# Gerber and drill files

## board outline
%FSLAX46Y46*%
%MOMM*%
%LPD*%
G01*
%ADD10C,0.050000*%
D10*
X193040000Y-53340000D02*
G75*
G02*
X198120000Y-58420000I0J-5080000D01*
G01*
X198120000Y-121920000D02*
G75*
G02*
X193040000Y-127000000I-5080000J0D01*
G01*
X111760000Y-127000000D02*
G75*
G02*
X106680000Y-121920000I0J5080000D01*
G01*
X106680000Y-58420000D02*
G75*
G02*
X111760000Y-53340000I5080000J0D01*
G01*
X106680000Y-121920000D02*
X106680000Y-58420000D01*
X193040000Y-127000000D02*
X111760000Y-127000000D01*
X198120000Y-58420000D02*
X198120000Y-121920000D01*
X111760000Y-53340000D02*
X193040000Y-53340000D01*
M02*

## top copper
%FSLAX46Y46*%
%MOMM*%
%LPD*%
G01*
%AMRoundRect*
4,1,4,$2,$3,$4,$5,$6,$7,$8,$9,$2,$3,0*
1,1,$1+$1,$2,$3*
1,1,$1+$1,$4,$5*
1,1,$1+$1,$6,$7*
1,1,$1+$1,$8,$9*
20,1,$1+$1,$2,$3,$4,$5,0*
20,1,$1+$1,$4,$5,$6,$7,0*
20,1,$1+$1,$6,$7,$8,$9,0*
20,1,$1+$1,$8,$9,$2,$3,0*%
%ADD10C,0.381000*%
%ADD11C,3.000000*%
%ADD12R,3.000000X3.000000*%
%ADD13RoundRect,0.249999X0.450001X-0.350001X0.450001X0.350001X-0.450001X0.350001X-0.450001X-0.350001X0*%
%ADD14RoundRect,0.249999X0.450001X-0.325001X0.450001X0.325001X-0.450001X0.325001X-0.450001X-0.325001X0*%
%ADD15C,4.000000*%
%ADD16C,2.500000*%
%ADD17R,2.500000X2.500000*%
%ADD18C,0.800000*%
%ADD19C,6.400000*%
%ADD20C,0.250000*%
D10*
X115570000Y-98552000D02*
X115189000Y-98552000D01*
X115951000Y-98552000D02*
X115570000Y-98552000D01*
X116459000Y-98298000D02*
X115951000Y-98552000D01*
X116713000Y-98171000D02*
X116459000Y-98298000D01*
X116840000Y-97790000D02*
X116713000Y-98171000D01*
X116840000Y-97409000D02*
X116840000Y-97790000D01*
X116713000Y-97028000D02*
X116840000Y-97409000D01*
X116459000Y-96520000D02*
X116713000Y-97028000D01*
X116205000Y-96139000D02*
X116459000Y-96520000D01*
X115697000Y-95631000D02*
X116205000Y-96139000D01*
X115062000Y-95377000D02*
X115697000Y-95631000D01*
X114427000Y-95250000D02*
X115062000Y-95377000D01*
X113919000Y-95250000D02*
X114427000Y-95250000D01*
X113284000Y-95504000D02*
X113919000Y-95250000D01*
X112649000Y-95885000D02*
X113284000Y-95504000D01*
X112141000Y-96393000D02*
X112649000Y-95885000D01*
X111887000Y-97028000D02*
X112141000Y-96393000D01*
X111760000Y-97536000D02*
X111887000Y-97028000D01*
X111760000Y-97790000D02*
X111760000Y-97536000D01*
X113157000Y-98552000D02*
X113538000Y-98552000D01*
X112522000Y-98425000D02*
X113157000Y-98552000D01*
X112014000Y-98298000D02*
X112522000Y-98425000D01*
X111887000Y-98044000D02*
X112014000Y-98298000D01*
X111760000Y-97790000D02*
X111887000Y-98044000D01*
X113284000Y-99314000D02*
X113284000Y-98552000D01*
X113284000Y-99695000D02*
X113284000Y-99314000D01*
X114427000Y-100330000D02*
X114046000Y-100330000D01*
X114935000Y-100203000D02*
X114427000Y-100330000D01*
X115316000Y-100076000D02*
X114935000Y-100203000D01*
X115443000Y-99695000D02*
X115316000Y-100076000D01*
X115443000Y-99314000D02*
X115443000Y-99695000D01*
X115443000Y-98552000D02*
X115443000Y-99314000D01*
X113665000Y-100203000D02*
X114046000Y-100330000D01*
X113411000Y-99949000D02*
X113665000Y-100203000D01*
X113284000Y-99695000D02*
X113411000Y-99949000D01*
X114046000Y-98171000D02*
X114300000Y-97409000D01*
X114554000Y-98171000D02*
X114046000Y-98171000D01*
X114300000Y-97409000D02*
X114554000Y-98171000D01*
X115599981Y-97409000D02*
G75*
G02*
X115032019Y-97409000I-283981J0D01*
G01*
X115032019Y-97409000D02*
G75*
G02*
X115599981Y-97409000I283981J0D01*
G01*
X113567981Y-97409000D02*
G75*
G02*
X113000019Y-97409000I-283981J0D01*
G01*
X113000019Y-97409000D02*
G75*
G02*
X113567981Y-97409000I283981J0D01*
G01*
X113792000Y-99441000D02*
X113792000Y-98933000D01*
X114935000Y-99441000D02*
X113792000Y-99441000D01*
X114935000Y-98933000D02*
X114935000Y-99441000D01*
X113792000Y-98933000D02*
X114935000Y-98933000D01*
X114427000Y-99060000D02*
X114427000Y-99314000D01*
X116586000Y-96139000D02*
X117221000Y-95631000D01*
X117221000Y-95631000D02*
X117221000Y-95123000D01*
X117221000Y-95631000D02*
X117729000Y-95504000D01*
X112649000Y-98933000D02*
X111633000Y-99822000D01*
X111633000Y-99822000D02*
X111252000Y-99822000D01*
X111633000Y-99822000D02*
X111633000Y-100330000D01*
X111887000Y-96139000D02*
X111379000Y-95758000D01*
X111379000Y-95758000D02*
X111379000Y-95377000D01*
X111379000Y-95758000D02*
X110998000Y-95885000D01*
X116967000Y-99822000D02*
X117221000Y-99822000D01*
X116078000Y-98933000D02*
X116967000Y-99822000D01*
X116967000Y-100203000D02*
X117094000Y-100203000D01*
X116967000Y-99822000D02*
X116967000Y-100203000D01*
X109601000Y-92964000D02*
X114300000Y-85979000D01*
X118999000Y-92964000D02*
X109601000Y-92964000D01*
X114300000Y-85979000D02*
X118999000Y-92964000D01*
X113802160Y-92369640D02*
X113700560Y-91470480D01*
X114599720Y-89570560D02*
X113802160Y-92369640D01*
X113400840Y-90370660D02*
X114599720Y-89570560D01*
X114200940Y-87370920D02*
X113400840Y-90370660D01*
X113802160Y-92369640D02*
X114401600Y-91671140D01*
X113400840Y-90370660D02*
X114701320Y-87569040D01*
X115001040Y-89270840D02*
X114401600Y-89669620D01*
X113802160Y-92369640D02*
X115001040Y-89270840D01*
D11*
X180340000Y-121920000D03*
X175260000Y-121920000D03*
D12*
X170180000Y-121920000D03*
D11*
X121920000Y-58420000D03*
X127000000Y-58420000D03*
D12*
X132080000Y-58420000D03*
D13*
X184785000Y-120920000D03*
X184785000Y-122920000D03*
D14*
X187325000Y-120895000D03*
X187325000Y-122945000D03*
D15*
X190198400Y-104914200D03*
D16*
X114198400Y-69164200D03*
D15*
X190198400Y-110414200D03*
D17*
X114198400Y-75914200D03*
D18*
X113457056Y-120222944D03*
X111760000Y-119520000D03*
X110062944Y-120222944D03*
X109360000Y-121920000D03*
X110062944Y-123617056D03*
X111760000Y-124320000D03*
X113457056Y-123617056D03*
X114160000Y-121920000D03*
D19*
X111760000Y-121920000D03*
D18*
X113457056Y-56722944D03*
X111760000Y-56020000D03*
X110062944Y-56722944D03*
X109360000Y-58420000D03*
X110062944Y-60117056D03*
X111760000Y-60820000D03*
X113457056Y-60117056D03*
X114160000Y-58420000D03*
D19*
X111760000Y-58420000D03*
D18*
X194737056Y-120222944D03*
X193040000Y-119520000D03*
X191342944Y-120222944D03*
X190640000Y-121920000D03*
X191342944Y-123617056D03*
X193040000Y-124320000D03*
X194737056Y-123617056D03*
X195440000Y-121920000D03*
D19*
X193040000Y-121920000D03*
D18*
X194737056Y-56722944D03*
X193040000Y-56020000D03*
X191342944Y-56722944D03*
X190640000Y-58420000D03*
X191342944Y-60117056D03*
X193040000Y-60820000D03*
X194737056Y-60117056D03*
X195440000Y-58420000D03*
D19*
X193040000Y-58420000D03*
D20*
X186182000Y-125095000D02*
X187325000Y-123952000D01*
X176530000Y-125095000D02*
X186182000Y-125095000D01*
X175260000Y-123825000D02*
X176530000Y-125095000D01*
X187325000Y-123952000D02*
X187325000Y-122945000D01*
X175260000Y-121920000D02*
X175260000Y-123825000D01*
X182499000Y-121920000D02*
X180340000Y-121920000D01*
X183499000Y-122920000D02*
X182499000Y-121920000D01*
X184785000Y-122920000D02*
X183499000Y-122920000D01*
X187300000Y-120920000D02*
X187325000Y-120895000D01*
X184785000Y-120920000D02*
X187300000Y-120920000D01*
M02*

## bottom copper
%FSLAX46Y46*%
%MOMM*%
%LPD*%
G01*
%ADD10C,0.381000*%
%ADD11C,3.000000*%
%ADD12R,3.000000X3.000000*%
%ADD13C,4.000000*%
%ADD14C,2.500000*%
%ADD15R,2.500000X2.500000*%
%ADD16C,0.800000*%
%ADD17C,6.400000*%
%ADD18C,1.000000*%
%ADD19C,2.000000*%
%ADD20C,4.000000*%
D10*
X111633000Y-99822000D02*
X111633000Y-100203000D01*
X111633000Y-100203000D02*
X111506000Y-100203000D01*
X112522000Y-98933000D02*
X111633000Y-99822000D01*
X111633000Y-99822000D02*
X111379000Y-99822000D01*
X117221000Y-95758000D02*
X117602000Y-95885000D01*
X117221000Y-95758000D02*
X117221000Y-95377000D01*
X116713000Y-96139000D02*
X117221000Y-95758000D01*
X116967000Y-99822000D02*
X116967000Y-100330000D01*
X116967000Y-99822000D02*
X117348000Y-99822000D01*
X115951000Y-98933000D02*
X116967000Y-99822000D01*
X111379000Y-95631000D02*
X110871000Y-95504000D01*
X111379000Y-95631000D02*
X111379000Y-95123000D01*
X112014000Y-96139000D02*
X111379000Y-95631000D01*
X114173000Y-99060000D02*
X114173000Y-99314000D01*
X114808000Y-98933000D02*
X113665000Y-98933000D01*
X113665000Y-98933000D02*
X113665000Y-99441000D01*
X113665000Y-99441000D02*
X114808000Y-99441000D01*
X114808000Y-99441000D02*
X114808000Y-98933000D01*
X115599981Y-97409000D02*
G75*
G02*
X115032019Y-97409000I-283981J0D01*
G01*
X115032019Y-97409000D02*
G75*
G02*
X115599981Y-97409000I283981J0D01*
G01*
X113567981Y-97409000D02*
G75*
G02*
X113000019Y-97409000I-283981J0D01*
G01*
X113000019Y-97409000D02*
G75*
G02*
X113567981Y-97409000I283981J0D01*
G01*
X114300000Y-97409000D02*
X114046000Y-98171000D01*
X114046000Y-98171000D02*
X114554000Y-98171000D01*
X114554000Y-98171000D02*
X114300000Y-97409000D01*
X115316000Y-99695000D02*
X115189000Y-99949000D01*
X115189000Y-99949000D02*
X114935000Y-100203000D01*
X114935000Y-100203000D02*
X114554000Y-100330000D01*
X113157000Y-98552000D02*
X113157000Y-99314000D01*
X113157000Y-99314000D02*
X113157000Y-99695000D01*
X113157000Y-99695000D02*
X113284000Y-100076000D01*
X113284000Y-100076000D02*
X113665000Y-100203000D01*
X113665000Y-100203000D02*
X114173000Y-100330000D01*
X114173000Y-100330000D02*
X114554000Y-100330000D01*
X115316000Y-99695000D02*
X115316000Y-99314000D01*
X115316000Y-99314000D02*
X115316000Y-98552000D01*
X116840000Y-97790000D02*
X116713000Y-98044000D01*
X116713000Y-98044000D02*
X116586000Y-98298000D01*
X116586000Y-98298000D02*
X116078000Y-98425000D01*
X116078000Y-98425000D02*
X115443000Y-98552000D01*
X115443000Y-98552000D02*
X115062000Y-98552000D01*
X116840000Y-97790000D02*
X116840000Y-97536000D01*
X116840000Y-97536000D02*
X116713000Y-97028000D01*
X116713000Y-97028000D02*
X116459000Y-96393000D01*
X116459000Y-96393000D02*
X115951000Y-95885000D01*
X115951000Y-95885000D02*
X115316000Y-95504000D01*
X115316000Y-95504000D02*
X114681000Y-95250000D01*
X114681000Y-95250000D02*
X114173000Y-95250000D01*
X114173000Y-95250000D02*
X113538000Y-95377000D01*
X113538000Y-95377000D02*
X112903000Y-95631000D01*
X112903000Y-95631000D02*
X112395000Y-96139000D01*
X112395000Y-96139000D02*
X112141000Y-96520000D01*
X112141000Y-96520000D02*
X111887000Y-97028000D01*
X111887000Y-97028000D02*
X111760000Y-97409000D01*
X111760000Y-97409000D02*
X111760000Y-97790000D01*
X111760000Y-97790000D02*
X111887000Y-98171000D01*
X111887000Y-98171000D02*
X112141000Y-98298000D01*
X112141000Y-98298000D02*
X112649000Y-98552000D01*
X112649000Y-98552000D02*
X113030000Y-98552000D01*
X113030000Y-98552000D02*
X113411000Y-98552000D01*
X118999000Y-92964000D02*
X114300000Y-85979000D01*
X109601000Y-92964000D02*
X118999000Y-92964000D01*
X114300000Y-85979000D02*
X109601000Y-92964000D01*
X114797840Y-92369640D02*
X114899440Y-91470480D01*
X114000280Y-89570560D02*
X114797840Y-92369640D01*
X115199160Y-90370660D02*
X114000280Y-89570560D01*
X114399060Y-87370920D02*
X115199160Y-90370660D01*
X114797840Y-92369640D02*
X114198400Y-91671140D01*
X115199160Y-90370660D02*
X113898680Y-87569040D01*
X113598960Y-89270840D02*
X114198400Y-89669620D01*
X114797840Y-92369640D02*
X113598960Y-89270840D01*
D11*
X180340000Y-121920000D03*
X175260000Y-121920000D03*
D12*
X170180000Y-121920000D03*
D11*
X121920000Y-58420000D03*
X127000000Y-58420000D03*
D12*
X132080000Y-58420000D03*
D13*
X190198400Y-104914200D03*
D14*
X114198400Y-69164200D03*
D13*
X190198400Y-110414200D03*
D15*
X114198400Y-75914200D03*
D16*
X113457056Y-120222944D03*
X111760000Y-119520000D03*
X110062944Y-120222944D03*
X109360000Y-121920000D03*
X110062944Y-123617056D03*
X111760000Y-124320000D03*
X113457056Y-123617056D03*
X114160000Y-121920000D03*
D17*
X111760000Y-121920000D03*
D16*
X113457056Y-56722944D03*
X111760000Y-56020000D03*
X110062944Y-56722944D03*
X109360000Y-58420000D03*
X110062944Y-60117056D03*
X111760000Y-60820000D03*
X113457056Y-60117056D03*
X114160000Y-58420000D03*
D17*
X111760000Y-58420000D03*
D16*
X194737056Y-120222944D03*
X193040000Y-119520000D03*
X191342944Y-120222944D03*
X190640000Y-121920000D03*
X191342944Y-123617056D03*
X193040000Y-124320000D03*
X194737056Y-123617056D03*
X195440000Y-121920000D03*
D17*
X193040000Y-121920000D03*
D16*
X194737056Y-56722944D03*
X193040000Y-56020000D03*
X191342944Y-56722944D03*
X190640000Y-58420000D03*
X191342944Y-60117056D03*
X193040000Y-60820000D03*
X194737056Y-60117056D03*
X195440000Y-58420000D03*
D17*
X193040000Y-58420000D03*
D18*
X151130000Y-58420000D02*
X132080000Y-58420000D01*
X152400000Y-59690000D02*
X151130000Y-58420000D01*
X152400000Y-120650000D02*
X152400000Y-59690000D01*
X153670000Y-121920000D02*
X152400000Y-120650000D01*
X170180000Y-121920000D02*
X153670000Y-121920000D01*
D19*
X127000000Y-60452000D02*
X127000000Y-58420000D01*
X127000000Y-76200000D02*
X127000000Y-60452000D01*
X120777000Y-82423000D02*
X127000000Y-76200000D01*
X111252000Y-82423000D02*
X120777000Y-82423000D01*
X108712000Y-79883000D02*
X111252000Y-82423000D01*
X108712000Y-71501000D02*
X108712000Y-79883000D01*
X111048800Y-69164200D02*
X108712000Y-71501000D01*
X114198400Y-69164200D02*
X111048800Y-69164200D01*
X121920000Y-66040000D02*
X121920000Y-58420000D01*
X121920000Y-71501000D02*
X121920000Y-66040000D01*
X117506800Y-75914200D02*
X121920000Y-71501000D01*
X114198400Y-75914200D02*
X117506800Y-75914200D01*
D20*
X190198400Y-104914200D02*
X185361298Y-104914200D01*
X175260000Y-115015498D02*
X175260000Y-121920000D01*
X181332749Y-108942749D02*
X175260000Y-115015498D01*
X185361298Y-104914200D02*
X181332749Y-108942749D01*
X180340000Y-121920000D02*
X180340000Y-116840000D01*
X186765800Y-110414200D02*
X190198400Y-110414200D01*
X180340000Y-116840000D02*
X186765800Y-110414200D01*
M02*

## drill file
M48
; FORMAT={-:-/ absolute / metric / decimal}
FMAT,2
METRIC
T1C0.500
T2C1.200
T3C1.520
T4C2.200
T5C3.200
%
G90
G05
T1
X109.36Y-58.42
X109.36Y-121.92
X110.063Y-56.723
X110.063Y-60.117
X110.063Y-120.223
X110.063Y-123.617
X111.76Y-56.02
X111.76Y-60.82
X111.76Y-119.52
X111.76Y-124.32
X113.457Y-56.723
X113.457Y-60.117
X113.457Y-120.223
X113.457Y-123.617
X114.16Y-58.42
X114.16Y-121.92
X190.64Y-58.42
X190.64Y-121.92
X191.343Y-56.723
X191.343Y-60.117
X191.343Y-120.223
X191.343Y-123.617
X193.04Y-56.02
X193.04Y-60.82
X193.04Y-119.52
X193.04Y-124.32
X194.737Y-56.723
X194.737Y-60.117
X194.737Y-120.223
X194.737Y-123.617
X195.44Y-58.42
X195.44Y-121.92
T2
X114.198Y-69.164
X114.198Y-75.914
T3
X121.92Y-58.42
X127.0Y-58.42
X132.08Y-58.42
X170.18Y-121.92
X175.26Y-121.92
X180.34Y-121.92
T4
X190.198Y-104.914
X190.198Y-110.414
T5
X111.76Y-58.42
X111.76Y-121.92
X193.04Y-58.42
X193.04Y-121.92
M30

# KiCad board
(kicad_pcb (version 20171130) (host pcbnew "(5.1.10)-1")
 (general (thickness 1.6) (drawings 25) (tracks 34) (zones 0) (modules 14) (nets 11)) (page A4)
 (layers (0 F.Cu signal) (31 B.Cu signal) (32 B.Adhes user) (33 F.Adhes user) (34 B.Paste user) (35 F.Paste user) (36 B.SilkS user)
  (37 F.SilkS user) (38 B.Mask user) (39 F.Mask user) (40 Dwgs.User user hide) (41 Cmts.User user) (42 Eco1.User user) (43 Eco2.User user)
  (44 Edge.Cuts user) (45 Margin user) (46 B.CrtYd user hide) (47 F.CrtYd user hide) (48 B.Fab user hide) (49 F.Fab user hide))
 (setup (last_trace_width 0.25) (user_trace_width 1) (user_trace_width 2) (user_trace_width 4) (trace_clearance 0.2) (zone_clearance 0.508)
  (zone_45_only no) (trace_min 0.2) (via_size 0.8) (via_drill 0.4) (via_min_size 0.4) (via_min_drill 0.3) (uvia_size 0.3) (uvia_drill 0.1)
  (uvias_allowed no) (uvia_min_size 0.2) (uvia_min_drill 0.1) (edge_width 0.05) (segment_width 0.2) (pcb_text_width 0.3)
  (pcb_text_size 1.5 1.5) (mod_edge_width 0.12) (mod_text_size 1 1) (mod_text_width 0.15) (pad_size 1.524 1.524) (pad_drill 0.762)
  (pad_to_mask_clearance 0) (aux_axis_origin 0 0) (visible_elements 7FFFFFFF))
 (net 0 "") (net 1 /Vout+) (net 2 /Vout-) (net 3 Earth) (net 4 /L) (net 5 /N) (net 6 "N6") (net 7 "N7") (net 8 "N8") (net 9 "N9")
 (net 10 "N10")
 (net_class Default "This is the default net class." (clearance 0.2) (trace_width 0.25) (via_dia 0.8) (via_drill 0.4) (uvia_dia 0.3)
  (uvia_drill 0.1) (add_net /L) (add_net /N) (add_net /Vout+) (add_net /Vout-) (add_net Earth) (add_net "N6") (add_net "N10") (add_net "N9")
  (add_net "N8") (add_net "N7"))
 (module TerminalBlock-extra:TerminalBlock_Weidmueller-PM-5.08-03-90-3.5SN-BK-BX (layer F.Cu) (at 170.18 121.92)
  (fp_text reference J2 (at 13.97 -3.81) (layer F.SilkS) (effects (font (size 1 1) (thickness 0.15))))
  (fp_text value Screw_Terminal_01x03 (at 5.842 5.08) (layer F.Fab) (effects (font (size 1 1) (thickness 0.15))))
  (pad 3 thru_hole circle (at 10.16 0) (size 3 3) (drill 1.52) (layers *.Cu *.Mask) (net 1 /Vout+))
  (pad 2 thru_hole circle (at 5.08 0) (size 3 3) (drill 1.52) (layers *.Cu *.Mask) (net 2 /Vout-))
  (pad 1 thru_hole rect (at 0 0) (size 3 3) (drill 1.52) (layers *.Cu *.Mask) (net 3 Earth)))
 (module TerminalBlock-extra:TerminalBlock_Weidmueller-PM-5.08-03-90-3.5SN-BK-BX (layer F.Cu) (at 132.08 58.42 180)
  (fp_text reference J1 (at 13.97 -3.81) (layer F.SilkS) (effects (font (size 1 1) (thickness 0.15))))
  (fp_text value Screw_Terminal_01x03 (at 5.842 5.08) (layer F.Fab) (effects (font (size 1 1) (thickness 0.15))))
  (pad 3 thru_hole circle (at 10.16 0 180) (size 3 3) (drill 1.52) (layers *.Cu *.Mask) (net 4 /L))
  (pad 2 thru_hole circle (at 5.08 0 180) (size 3 3) (drill 1.52) (layers *.Cu *.Mask) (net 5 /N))
  (pad 1 thru_hole rect (at 0 0 180) (size 3 3) (drill 1.52) (layers *.Cu *.Mask) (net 3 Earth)))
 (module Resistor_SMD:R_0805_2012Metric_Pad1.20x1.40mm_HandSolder (layer F.Cu) (at 184.785 121.92 90)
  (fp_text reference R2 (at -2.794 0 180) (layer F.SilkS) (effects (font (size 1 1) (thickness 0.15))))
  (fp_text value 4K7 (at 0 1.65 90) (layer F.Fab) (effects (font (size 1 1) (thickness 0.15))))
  (pad 2 smd roundrect (at 1 0 90) (size 1.2 1.4) (layers F.Cu F.Paste F.Mask) (roundrect_rratio 0.2083325) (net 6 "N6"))
  (pad 1 smd roundrect (at -1 0 90) (size 1.2 1.4) (layers F.Cu F.Paste F.Mask) (roundrect_rratio 0.2083325) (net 1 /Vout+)))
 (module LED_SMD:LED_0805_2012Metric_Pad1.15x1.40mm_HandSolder (layer F.Cu) (at 187.325 121.92 90)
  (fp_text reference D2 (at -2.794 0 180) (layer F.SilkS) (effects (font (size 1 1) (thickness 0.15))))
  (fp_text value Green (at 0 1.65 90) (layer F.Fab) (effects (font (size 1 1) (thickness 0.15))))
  (pad 2 smd roundrect (at 1.025 0 90) (size 1.15 1.4) (layers F.Cu F.Paste F.Mask) (roundrect_rratio 0.2173904347826087) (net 6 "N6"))
  (pad 1 smd roundrect (at -1.025 0 90) (size 1.15 1.4) (layers F.Cu F.Paste F.Mask) (roundrect_rratio 0.2173904347826087) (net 2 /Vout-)))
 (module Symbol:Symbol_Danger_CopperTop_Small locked (layer B.Cu) (at 114.3 97.79 180)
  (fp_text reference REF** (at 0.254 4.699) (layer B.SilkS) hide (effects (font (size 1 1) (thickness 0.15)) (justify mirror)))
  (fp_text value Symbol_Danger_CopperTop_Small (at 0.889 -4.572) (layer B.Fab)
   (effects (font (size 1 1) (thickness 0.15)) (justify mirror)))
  (fp_line (start 2.667 -2.032) (end 2.667 -2.413) (layer B.Cu) (width 0.381))
  (fp_line (start 2.667 -2.413) (end 2.794 -2.413) (layer B.Cu) (width 0.381))
  (fp_line (start 1.778 -1.143) (end 2.667 -2.032) (layer B.Cu) (width 0.381))
  (fp_line (start 2.667 -2.032) (end 2.921 -2.032) (layer B.Cu) (width 0.381))
  (fp_line (start -2.921 2.032) (end -3.302 1.905) (layer B.Cu) (width 0.381))
  (fp_line (start -2.921 2.032) (end -2.921 2.413) (layer B.Cu) (width 0.381))
  (fp_line (start -2.413 1.651) (end -2.921 2.032) (layer B.Cu) (width 0.381))
  (fp_line (start -2.667 -2.032) (end -2.667 -2.54) (layer B.Cu) (width 0.381))
  (fp_line (start -2.667 -2.032) (end -3.048 -2.032) (layer B.Cu) (width 0.381))
  (fp_line (start -1.651 -1.143) (end -2.667 -2.032) (layer B.Cu) (width 0.381))
  (fp_line (start 2.921 2.159) (end 3.429 2.286) (layer B.Cu) (width 0.381))
  (fp_line (start 2.921 2.159) (end 2.921 2.667) (layer B.Cu) (width 0.381))
  (fp_line (start 2.286 1.651) (end 2.921 2.159) (layer B.Cu) (width 0.381))
  (fp_line (start 0.127 -1.27) (end 0.127 -1.524) (layer B.Cu) (width 0.381))
  (fp_line (start -0.508 -1.143) (end 0.635 -1.143) (layer B.Cu) (width 0.381))
  (fp_line (start 0.635 -1.143) (end 0.635 -1.651) (layer B.Cu) (width 0.381))
  (fp_line (start 0.635 -1.651) (end -0.508 -1.651) (layer B.Cu) (width 0.381))
  (fp_line (start -0.508 -1.651) (end -0.508 -1.143) (layer B.Cu) (width 0.381))
  (fp_circle (center -1.016 0.381) (end -1.27 0.254) (layer B.Cu) (width 0.381))
  (fp_circle (center 1.016 0.381) (end 1.27 0.254) (layer B.Cu) (width 0.381))
  (fp_line (start 0 0.381) (end 0.254 -0.381) (layer B.Cu) (width 0.381))
  (fp_line (start 0.254 -0.381) (end -0.254 -0.381) (layer B.Cu) (width 0.381))
  (fp_line (start -0.254 -0.381) (end 0 0.381) (layer B.Cu) (width 0.381))
  (fp_line (start -1.016 -1.905) (end -0.889 -2.159) (layer B.Cu) (width 0.381))
  (fp_line (start -0.889 -2.159) (end -0.635 -2.413) (layer B.Cu) (width 0.381))
  (fp_line (start -0.635 -2.413) (end -0.254 -2.54) (layer B.Cu) (width 0.381))
  (fp_line (start 1.143 -0.762) (end 1.143 -1.524) (layer B.Cu) (width 0.381))
  (fp_line (start 1.143 -1.524) (end 1.143 -1.905) (layer B.Cu) (width 0.381))
  (fp_line (start 1.143 -1.905) (end 1.016 -2.286) (layer B.Cu) (width 0.381))
  (fp_line (start 1.016 -2.286) (end 0.635 -2.413) (layer B.Cu) (width 0.381))
  (fp_line (start 0.635 -2.413) (end 0.127 -2.54) (layer B.Cu) (width 0.381))
  (fp_line (start 0.127 -2.54) (end -0.254 -2.54) (layer B.Cu) (width 0.381))
  (fp_line (start -1.016 -1.905) (end -1.016 -1.524) (layer B.Cu) (width 0.381))
  (fp_line (start -1.016 -1.524) (end -1.016 -0.762) (layer B.Cu) (width 0.381))
  (fp_line (start -2.54 0) (end -2.413 -0.254) (layer B.Cu) (width 0.381))
  (fp_line (start -2.413 -0.254) (end -2.286 -0.508) (layer B.Cu) (width 0.381))
  (fp_line (start -2.286 -0.508) (end -1.778 -0.635) (layer B.Cu) (width 0.381))
  (fp_line (start -1.778 -0.635) (end -1.143 -0.762) (layer B.Cu) (width 0.381))
  (fp_line (start -1.143 -0.762) (end -0.762 -0.762) (layer B.Cu) (width 0.381))
  (fp_line (start -2.54 0) (end -2.54 0.254) (layer B.Cu) (width 0.381))
  (fp_line (start -2.54 0.254) (end -2.413 0.762) (layer B.Cu) (width 0.381))
  (fp_line (start -2.413 0.762) (end -2.159 1.397) (layer B.Cu) (width 0.381))
  (fp_line (start -2.159 1.397) (end -1.651 1.905) (layer B.Cu) (width 0.381))
  (fp_line (start -1.651 1.905) (end -1.016 2.286) (layer B.Cu) (width 0.381))
  (fp_line (start -1.016 2.286) (end -0.381 2.54) (layer B.Cu) (width 0.381))
  (fp_line (start -0.381 2.54) (end 0.127 2.54) (layer B.Cu) (width 0.381))
  (fp_line (start 0.127 2.54) (end 0.762 2.413) (layer B.Cu) (width 0.381))
  (fp_line (start 0.762 2.413) (end 1.397 2.159) (layer B.Cu) (width 0.381))
  (fp_line (start 1.397 2.159) (end 1.905 1.651) (layer B.Cu) (width 0.381))
  (fp_line (start 1.905 1.651) (end 2.159 1.27) (layer B.Cu) (width 0.381))
  (fp_line (start 2.159 1.27) (end 2.413 0.762) (layer B.Cu) (width 0.381))
  (fp_line (start 2.413 0.762) (end 2.54 0.381) (layer B.Cu) (width 0.381))
  (fp_line (start 2.54 0.381) (end 2.54 0) (layer B.Cu) (width 0.381))
  (fp_line (start 2.54 0) (end 2.413 -0.381) (layer B.Cu) (width 0.381))
  (fp_line (start 2.413 -0.381) (end 2.159 -0.508) (layer B.Cu) (width 0.381))
  (fp_line (start 2.159 -0.508) (end 1.651 -0.762) (layer B.Cu) (width 0.381))
  (fp_line (start 1.651 -0.762) (end 1.27 -0.762) (layer B.Cu) (width 0.381))
  (fp_line (start 1.27 -0.762) (end 0.889 -0.762) (layer B.Cu) (width 0.381)))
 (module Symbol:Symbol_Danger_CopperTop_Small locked (layer F.Cu) (at 114.3 97.79)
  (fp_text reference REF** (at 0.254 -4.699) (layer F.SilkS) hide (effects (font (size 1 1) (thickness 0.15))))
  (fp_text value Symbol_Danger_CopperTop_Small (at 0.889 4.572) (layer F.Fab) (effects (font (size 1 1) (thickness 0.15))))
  (fp_line (start 1.27 0.762) (end 0.889 0.762) (layer F.Cu) (width 0.381))
  (fp_line (start 1.651 0.762) (end 1.27 0.762) (layer F.Cu) (width 0.381))
  (fp_line (start 2.159 0.508) (end 1.651 0.762) (layer F.Cu) (width 0.381))
  (fp_line (start 2.413 0.381) (end 2.159 0.508) (layer F.Cu) (width 0.381))
  (fp_line (start 2.54 0) (end 2.413 0.381) (layer F.Cu) (width 0.381))
  (fp_line (start 2.54 -0.381) (end 2.54 0) (layer F.Cu) (width 0.381))
  (fp_line (start 2.413 -0.762) (end 2.54 -0.381) (layer F.Cu) (width 0.381))
  (fp_line (start 2.159 -1.27) (end 2.413 -0.762) (layer F.Cu) (width 0.381))
  (fp_line (start 1.905 -1.651) (end 2.159 -1.27) (layer F.Cu) (width 0.381))
  (fp_line (start 1.397 -2.159) (end 1.905 -1.651) (layer F.Cu) (width 0.381))
  (fp_line (start 0.762 -2.413) (end 1.397 -2.159) (layer F.Cu) (width 0.381))
  (fp_line (start 0.127 -2.54) (end 0.762 -2.413) (layer F.Cu) (width 0.381))
  (fp_line (start -0.381 -2.54) (end 0.127 -2.54) (layer F.Cu) (width 0.381))
  (fp_line (start -1.016 -2.286) (end -0.381 -2.54) (layer F.Cu) (width 0.381))
  (fp_line (start -1.651 -1.905) (end -1.016 -2.286) (layer F.Cu) (width 0.381))
  (fp_line (start -2.159 -1.397) (end -1.651 -1.905) (layer F.Cu) (width 0.381))
  (fp_line (start -2.413 -0.762) (end -2.159 -1.397) (layer F.Cu) (width 0.381))
  (fp_line (start -2.54 -0.254) (end -2.413 -0.762) (layer F.Cu) (width 0.381))
  (fp_line (start -2.54 0) (end -2.54 -0.254) (layer F.Cu) (width 0.381))
  (fp_line (start -1.143 0.762) (end -0.762 0.762) (layer F.Cu) (width 0.381))
  (fp_line (start -1.778 0.635) (end -1.143 0.762) (layer F.Cu) (width 0.381))
  (fp_line (start -2.286 0.508) (end -1.778 0.635) (layer F.Cu) (width 0.381))
  (fp_line (start -2.413 0.254) (end -2.286 0.508) (layer F.Cu) (width 0.381))
  (fp_line (start -2.54 0) (end -2.413 0.254) (layer F.Cu) (width 0.381))
  (fp_line (start -1.016 1.524) (end -1.016 0.762) (layer F.Cu) (width 0.381))
  (fp_line (start -1.016 1.905) (end -1.016 1.524) (layer F.Cu) (width 0.381))
  (fp_line (start 0.127 2.54) (end -0.254 2.54) (layer F.Cu) (width 0.381))
  (fp_line (start 0.635 2.413) (end 0.127 2.54) (layer F.Cu) (width 0.381))
  (fp_line (start 1.016 2.286) (end 0.635 2.413) (layer F.Cu) (width 0.381))
  (fp_line (start 1.143 1.905) (end 1.016 2.286) (layer F.Cu) (width 0.381))
  (fp_line (start 1.143 1.524) (end 1.143 1.905) (layer F.Cu) (width 0.381))
  (fp_line (start 1.143 0.762) (end 1.143 1.524) (layer F.Cu) (width 0.381))
  (fp_line (start -0.635 2.413) (end -0.254 2.54) (layer F.Cu) (width 0.381))
  (fp_line (start -0.889 2.159) (end -0.635 2.413) (layer F.Cu) (width 0.381))
  (fp_line (start -1.016 1.905) (end -0.889 2.159) (layer F.Cu) (width 0.381))
  (fp_line (start -0.254 0.381) (end 0 -0.381) (layer F.Cu) (width 0.381))
  (fp_line (start 0.254 0.381) (end -0.254 0.381) (layer F.Cu) (width 0.381))
  (fp_line (start 0 -0.381) (end 0.254 0.381) (layer F.Cu) (width 0.381))
  (fp_circle (center 1.016 -0.381) (end 1.27 -0.254) (layer F.Cu) (width 0.381))
  (fp_circle (center -1.016 -0.381) (end -1.27 -0.254) (layer F.Cu) (width 0.381))
  (fp_line (start -0.508 1.651) (end -0.508 1.143) (layer F.Cu) (width 0.381))
  (fp_line (start 0.635 1.651) (end -0.508 1.651) (layer F.Cu) (width 0.381))
  (fp_line (start 0.635 1.143) (end 0.635 1.651) (layer F.Cu) (width 0.381))
  (fp_line (start -0.508 1.143) (end 0.635 1.143) (layer F.Cu) (width 0.381))
  (fp_line (start 0.127 1.27) (end 0.127 1.524) (layer F.Cu) (width 0.381))
  (fp_line (start 2.286 -1.651) (end 2.921 -2.159) (layer F.Cu) (width 0.381))
  (fp_line (start 2.921 -2.159) (end 2.921 -2.667) (layer F.Cu) (width 0.381))
  (fp_line (start 2.921 -2.159) (end 3.429 -2.286) (layer F.Cu) (width 0.381))
  (fp_line (start -1.651 1.143) (end -2.667 2.032) (layer F.Cu) (width 0.381))
  (fp_line (start -2.667 2.032) (end -3.048 2.032) (layer F.Cu) (width 0.381))
  (fp_line (start -2.667 2.032) (end -2.667 2.54) (layer F.Cu) (width 0.381))
  (fp_line (start -2.413 -1.651) (end -2.921 -2.032) (layer F.Cu) (width 0.381))
  (fp_line (start -2.921 -2.032) (end -2.921 -2.413) (layer F.Cu) (width 0.381))
  (fp_line (start -2.921 -2.032) (end -3.302 -1.905) (layer F.Cu) (width 0.381))
  (fp_line (start 2.667 2.032) (end 2.921 2.032) (layer F.Cu) (width 0.381))
  (fp_line (start 1.778 1.143) (end 2.667 2.032) (layer F.Cu) (width 0.381))
  (fp_line (start 2.667 2.413) (end 2.794 2.413) (layer F.Cu) (width 0.381))
  (fp_line (start 2.667 2.032) (end 2.667 2.413) (layer F.Cu) (width 0.381)))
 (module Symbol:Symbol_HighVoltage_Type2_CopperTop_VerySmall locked (layer B.Cu) (at 114.3 90.17 180)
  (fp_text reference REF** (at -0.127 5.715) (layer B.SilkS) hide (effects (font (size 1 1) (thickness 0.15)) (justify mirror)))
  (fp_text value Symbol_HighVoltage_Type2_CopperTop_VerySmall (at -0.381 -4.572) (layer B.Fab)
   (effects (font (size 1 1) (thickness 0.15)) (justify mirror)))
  (fp_line (start -4.699 -2.794) (end 0 4.191) (layer B.Cu) (width 0.381))
  (fp_line (start 4.699 -2.794) (end -4.699 -2.794) (layer B.Cu) (width 0.381))
  (fp_line (start 0 4.191) (end 4.699 -2.794) (layer B.Cu) (width 0.381))
  (fp_line (start -0.49784 -2.19964) (end -0.59944 -1.30048) (layer B.Cu) (width 0.381))
  (fp_line (start 0.29972 0.59944) (end -0.49784 -2.19964) (layer B.Cu) (width 0.381))
  (fp_line (start -0.89916 -0.20066) (end 0.29972 0.59944) (layer B.Cu) (width 0.381))
  (fp_line (start -0.09906 2.79908) (end -0.89916 -0.20066) (layer B.Cu) (width 0.381))
  (fp_line (start -0.49784 -2.19964) (end 0.1016 -1.50114) (layer B.Cu) (width 0.381))
  (fp_line (start -0.89916 -0.20066) (end 0.40132 2.60096) (layer B.Cu) (width 0.381))
  (fp_line (start 0.70104 0.89916) (end 0.1016 0.50038) (layer B.Cu) (width 0.381))
  (fp_line (start -0.49784 -2.19964) (end 0.70104 0.89916) (layer B.Cu) (width 0.381)))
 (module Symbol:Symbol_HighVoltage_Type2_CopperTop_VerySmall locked (layer F.Cu) (at 114.3 90.17)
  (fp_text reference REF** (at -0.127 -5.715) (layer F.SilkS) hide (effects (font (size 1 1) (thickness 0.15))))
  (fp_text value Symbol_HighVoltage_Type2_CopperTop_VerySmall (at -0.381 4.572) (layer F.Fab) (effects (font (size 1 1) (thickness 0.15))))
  (fp_line (start -4.699 2.794) (end 0 -4.191) (layer F.Cu) (width 0.381))
  (fp_line (start 4.699 2.794) (end -4.699 2.794) (layer F.Cu) (width 0.381))
  (fp_line (start 0 -4.191) (end 4.699 2.794) (layer F.Cu) (width 0.381))
  (fp_line (start -0.49784 2.19964) (end -0.59944 1.30048) (layer F.Cu) (width 0.381))
  (fp_line (start 0.29972 -0.59944) (end -0.49784 2.19964) (layer F.Cu) (width 0.381))
  (fp_line (start -0.89916 0.20066) (end 0.29972 -0.59944) (layer F.Cu) (width 0.381))
  (fp_line (start -0.09906 -2.79908) (end -0.89916 0.20066) (layer F.Cu) (width 0.381))
  (fp_line (start -0.49784 2.19964) (end 0.1016 1.50114) (layer F.Cu) (width 0.381))
  (fp_line (start -0.89916 0.20066) (end 0.40132 -2.60096) (layer F.Cu) (width 0.381))
  (fp_line (start 0.70104 -0.89916) (end 0.1016 -0.50038) (layer F.Cu) (width 0.381))
  (fp_line (start -0.49784 2.19964) (end 0.70104 -0.89916) (layer F.Cu) (width 0.381)))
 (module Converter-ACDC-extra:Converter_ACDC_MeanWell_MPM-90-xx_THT (layer F.Cu) (at 152.4 90.17)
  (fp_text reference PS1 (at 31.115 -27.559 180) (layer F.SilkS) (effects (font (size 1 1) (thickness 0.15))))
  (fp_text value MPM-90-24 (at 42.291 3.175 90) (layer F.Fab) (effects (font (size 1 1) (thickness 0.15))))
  (pad 4 thru_hole circle (at 37.7984 14.7442) (size 4 4) (drill 2.2) (layers *.Cu *.Mask) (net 2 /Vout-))
  (pad 2 thru_hole circle (at -38.2016 -21.0058) (size 2.5 2.5) (drill 1.2) (layers *.Cu *.Mask) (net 5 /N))
  (pad 3 thru_hole circle (at 37.7984 20.2442) (size 4 4) (drill 2.2) (layers *.Cu *.Mask) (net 1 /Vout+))
  (pad 1 thru_hole rect (at -38.2016 -14.2558) (size 2.5 2.5) (drill 1.2) (layers *.Cu *.Mask) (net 4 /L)))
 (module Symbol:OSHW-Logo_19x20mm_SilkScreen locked (layer B.Cu) (at 152.4 109.22 180)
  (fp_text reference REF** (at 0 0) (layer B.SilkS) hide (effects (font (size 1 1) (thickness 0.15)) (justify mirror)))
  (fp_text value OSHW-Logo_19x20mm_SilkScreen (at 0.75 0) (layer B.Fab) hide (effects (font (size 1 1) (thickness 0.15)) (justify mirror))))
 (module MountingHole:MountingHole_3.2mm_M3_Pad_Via (layer F.Cu) (at 111.76 121.92)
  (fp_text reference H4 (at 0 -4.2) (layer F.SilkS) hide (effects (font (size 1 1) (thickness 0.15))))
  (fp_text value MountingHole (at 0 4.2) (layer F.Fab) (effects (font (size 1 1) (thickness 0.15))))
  (pad 1 thru_hole circle (at 1.697056 -1.697056) (size 0.8 0.8) (drill 0.5) (layers *.Cu *.Mask) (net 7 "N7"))
  (pad 1 thru_hole circle (at 0 -2.4) (size 0.8 0.8) (drill 0.5) (layers *.Cu *.Mask) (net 7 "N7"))
  (pad 1 thru_hole circle (at -1.697056 -1.697056) (size 0.8 0.8) (drill 0.5) (layers *.Cu *.Mask) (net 7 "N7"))
  (pad 1 thru_hole circle (at -2.4 0) (size 0.8 0.8) (drill 0.5) (layers *.Cu *.Mask) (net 7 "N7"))
  (pad 1 thru_hole circle (at -1.697056 1.697056) (size 0.8 0.8) (drill 0.5) (layers *.Cu *.Mask) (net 7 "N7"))
  (pad 1 thru_hole circle (at 0 2.4) (size 0.8 0.8) (drill 0.5) (layers *.Cu *.Mask) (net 7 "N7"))
  (pad 1 thru_hole circle (at 1.697056 1.697056) (size 0.8 0.8) (drill 0.5) (layers *.Cu *.Mask) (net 7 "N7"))
  (pad 1 thru_hole circle (at 2.4 0) (size 0.8 0.8) (drill 0.5) (layers *.Cu *.Mask) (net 7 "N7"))
  (pad 1 thru_hole circle (at 0 0) (size 6.4 6.4) (drill 3.2) (layers *.Cu *.Mask) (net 7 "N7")))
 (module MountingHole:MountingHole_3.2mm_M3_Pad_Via (layer F.Cu) (at 111.76 58.42)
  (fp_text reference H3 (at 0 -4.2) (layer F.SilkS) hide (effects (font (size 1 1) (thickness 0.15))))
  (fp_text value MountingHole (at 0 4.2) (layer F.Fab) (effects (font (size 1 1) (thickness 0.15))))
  (pad 1 thru_hole circle (at 1.697056 -1.697056) (size 0.8 0.8) (drill 0.5) (layers *.Cu *.Mask) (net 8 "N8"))
  (pad 1 thru_hole circle (at 0 -2.4) (size 0.8 0.8) (drill 0.5) (layers *.Cu *.Mask) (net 8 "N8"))
  (pad 1 thru_hole circle (at -1.697056 -1.697056) (size 0.8 0.8) (drill 0.5) (layers *.Cu *.Mask) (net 8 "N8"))
  (pad 1 thru_hole circle (at -2.4 0) (size 0.8 0.8) (drill 0.5) (layers *.Cu *.Mask) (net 8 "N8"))
  (pad 1 thru_hole circle (at -1.697056 1.697056) (size 0.8 0.8) (drill 0.5) (layers *.Cu *.Mask) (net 8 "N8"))
  (pad 1 thru_hole circle (at 0 2.4) (size 0.8 0.8) (drill 0.5) (layers *.Cu *.Mask) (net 8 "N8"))
  (pad 1 thru_hole circle (at 1.697056 1.697056) (size 0.8 0.8) (drill 0.5) (layers *.Cu *.Mask) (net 8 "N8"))
  (pad 1 thru_hole circle (at 2.4 0) (size 0.8 0.8) (drill 0.5) (layers *.Cu *.Mask) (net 8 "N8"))
  (pad 1 thru_hole circle (at 0 0) (size 6.4 6.4) (drill 3.2) (layers *.Cu *.Mask) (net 8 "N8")))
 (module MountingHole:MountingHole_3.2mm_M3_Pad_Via (layer F.Cu) (at 193.04 121.92)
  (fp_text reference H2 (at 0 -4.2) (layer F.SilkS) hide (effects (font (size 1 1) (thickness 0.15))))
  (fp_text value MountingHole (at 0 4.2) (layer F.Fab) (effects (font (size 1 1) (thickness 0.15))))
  (pad 1 thru_hole circle (at 1.697056 -1.697056) (size 0.8 0.8) (drill 0.5) (layers *.Cu *.Mask) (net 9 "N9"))
  (pad 1 thru_hole circle (at 0 -2.4) (size 0.8 0.8) (drill 0.5) (layers *.Cu *.Mask) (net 9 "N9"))
  (pad 1 thru_hole circle (at -1.697056 -1.697056) (size 0.8 0.8) (drill 0.5) (layers *.Cu *.Mask) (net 9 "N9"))
  (pad 1 thru_hole circle (at -2.4 0) (size 0.8 0.8) (drill 0.5) (layers *.Cu *.Mask) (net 9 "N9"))
  (pad 1 thru_hole circle (at -1.697056 1.697056) (size 0.8 0.8) (drill 0.5) (layers *.Cu *.Mask) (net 9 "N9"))
  (pad 1 thru_hole circle (at 0 2.4) (size 0.8 0.8) (drill 0.5) (layers *.Cu *.Mask) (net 9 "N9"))
  (pad 1 thru_hole circle (at 1.697056 1.697056) (size 0.8 0.8) (drill 0.5) (layers *.Cu *.Mask) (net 9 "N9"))
  (pad 1 thru_hole circle (at 2.4 0) (size 0.8 0.8) (drill 0.5) (layers *.Cu *.Mask) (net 9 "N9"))
  (pad 1 thru_hole circle (at 0 0) (size 6.4 6.4) (drill 3.2) (layers *.Cu *.Mask) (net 9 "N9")))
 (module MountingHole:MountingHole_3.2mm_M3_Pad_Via (layer F.Cu) (at 193.04 58.42)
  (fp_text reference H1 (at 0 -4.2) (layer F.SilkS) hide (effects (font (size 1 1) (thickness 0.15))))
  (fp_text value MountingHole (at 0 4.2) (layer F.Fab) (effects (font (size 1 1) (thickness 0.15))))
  (pad 1 thru_hole circle (at 1.697056 -1.697056) (size 0.8 0.8) (drill 0.5) (layers *.Cu *.Mask) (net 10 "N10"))
  (pad 1 thru_hole circle (at 0 -2.4) (size 0.8 0.8) (drill 0.5) (layers *.Cu *.Mask) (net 10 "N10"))
  (pad 1 thru_hole circle (at -1.697056 -1.697056) (size 0.8 0.8) (drill 0.5) (layers *.Cu *.Mask) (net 10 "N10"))
  (pad 1 thru_hole circle (at -2.4 0) (size 0.8 0.8) (drill 0.5) (layers *.Cu *.Mask) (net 10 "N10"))
  (pad 1 thru_hole circle (at -1.697056 1.697056) (size 0.8 0.8) (drill 0.5) (layers *.Cu *.Mask) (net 10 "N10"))
  (pad 1 thru_hole circle (at 0 2.4) (size 0.8 0.8) (drill 0.5) (layers *.Cu *.Mask) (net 10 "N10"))
  (pad 1 thru_hole circle (at 1.697056 1.697056) (size 0.8 0.8) (drill 0.5) (layers *.Cu *.Mask) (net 10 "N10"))
  (pad 1 thru_hole circle (at 2.4 0) (size 0.8 0.8) (drill 0.5) (layers *.Cu *.Mask) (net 10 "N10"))
  (pad 1 thru_hole circle (at 0 0) (size 6.4 6.4) (drill 3.2) (layers *.Cu *.Mask) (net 10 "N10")))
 (gr_arc (start 193.04 58.42) (end 198.12 58.42) (angle -90) (layer Edge.Cuts) (width 0.05))
 (gr_arc (start 193.04 121.92) (end 193.04 127) (angle -90) (layer Edge.Cuts) (width 0.05))
 (gr_arc (start 111.76 121.92) (end 106.68 121.92) (angle -90) (layer Edge.Cuts) (width 0.05))
 (gr_arc (start 111.76 58.42) (end 111.76 53.34) (angle -90) (layer Edge.Cuts) (width 0.05))
 (gr_line (start 106.68 121.92) (end 106.68 58.42) (layer Edge.Cuts) (width 0.05))
 (gr_line (start 193.04 127) (end 111.76 127) (layer Edge.Cuts) (width 0.05))
 (gr_line (start 198.12 58.42) (end 198.12 121.92) (layer Edge.Cuts) (width 0.05))
 (gr_line (start 111.76 53.34) (end 193.04 53.34) (layer Edge.Cuts) (width 0.05))
 (segment (start 151.13 58.42) (end 132.08 58.42) (width 1) (layer B.Cu) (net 3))
 (segment (start 152.4 59.69) (end 151.13 58.42) (width 1) (layer B.Cu) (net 3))
 (segment (start 152.4 120.65) (end 152.4 59.69) (width 1) (layer B.Cu) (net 3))
 (segment (start 153.67 121.92) (end 152.4 120.65) (width 1) (layer B.Cu) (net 3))
 (segment (start 170.18 121.92) (end 153.67 121.92) (width 1) (layer B.Cu) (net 3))
 (segment (start 127 60.452) (end 127 58.42) (width 2) (layer B.Cu) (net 5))
 (segment (start 127 76.2) (end 127 60.452) (width 2) (layer B.Cu) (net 5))
 (segment (start 120.777 82.423) (end 127 76.2) (width 2) (layer B.Cu) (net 5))
 (segment (start 111.252 82.423) (end 120.777 82.423) (width 2) (layer B.Cu) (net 5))
 (segment (start 108.712 79.883) (end 111.252 82.423) (width 2) (layer B.Cu) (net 5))
 (segment (start 108.712 71.501) (end 108.712 79.883) (width 2) (layer B.Cu) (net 5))
 (segment (start 111.0488 69.1642) (end 108.712 71.501) (width 2) (layer B.Cu) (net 5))
 (segment (start 114.1984 69.1642) (end 111.0488 69.1642) (width 2) (layer B.Cu) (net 5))
 (segment (start 121.92 66.04) (end 121.92 58.42) (width 2) (layer B.Cu) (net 4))
 (segment (start 121.92 71.501) (end 121.92 66.04) (width 2) (layer B.Cu) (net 4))
 (segment (start 117.5068 75.9142) (end 121.92 71.501) (width 2) (layer B.Cu) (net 4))
 (segment (start 114.1984 75.9142) (end 117.5068 75.9142) (width 2) (layer B.Cu) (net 4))
 (segment (start 190.1984 104.9142) (end 185.361298 104.9142) (width 4) (layer B.Cu) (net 2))
 (segment (start 175.26 115.015498) (end 175.26 121.92) (width 4) (layer B.Cu) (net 2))
 (segment (start 181.332749 108.942749) (end 175.26 115.015498) (width 4) (layer B.Cu) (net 2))
 (segment (start 185.361298 104.9142) (end 181.332749 108.942749) (width 4) (layer B.Cu) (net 2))
 (segment (start 186.182 125.095) (end 187.325 123.952) (width 0.25) (layer F.Cu) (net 2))
 (segment (start 176.53 125.095) (end 186.182 125.095) (width 0.25) (layer F.Cu) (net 2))
 (segment (start 175.26 123.825) (end 176.53 125.095) (width 0.25) (layer F.Cu) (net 2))
 (segment (start 187.325 123.952) (end 187.325 122.945) (width 0.25) (layer F.Cu) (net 2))
 (segment (start 175.26 121.92) (end 175.26 123.825) (width 0.25) (layer F.Cu) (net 2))
 (segment (start 180.34 121.92) (end 180.34 116.84) (width 4) (layer B.Cu) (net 1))
 (segment (start 186.7658 110.4142) (end 190.1984 110.4142) (width 4) (layer B.Cu) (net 1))
 (segment (start 180.34 116.84) (end 186.7658 110.4142) (width 4) (layer B.Cu) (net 1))
 (segment (start 182.499 121.92) (end 180.34 121.92) (width 0.25) (layer F.Cu) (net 1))
 (segment (start 183.499 122.92) (end 182.499 121.92) (width 0.25) (layer F.Cu) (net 1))
 (segment (start 184.785 122.92) (end 183.499 122.92) (width 0.25) (layer F.Cu) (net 1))
 (segment (start 187.3 120.92) (end 187.325 120.895) (width 0.25) (layer F.Cu) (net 6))
 (segment (start 184.785 120.92) (end 187.3 120.92) (width 0.25) (layer F.Cu) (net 6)))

